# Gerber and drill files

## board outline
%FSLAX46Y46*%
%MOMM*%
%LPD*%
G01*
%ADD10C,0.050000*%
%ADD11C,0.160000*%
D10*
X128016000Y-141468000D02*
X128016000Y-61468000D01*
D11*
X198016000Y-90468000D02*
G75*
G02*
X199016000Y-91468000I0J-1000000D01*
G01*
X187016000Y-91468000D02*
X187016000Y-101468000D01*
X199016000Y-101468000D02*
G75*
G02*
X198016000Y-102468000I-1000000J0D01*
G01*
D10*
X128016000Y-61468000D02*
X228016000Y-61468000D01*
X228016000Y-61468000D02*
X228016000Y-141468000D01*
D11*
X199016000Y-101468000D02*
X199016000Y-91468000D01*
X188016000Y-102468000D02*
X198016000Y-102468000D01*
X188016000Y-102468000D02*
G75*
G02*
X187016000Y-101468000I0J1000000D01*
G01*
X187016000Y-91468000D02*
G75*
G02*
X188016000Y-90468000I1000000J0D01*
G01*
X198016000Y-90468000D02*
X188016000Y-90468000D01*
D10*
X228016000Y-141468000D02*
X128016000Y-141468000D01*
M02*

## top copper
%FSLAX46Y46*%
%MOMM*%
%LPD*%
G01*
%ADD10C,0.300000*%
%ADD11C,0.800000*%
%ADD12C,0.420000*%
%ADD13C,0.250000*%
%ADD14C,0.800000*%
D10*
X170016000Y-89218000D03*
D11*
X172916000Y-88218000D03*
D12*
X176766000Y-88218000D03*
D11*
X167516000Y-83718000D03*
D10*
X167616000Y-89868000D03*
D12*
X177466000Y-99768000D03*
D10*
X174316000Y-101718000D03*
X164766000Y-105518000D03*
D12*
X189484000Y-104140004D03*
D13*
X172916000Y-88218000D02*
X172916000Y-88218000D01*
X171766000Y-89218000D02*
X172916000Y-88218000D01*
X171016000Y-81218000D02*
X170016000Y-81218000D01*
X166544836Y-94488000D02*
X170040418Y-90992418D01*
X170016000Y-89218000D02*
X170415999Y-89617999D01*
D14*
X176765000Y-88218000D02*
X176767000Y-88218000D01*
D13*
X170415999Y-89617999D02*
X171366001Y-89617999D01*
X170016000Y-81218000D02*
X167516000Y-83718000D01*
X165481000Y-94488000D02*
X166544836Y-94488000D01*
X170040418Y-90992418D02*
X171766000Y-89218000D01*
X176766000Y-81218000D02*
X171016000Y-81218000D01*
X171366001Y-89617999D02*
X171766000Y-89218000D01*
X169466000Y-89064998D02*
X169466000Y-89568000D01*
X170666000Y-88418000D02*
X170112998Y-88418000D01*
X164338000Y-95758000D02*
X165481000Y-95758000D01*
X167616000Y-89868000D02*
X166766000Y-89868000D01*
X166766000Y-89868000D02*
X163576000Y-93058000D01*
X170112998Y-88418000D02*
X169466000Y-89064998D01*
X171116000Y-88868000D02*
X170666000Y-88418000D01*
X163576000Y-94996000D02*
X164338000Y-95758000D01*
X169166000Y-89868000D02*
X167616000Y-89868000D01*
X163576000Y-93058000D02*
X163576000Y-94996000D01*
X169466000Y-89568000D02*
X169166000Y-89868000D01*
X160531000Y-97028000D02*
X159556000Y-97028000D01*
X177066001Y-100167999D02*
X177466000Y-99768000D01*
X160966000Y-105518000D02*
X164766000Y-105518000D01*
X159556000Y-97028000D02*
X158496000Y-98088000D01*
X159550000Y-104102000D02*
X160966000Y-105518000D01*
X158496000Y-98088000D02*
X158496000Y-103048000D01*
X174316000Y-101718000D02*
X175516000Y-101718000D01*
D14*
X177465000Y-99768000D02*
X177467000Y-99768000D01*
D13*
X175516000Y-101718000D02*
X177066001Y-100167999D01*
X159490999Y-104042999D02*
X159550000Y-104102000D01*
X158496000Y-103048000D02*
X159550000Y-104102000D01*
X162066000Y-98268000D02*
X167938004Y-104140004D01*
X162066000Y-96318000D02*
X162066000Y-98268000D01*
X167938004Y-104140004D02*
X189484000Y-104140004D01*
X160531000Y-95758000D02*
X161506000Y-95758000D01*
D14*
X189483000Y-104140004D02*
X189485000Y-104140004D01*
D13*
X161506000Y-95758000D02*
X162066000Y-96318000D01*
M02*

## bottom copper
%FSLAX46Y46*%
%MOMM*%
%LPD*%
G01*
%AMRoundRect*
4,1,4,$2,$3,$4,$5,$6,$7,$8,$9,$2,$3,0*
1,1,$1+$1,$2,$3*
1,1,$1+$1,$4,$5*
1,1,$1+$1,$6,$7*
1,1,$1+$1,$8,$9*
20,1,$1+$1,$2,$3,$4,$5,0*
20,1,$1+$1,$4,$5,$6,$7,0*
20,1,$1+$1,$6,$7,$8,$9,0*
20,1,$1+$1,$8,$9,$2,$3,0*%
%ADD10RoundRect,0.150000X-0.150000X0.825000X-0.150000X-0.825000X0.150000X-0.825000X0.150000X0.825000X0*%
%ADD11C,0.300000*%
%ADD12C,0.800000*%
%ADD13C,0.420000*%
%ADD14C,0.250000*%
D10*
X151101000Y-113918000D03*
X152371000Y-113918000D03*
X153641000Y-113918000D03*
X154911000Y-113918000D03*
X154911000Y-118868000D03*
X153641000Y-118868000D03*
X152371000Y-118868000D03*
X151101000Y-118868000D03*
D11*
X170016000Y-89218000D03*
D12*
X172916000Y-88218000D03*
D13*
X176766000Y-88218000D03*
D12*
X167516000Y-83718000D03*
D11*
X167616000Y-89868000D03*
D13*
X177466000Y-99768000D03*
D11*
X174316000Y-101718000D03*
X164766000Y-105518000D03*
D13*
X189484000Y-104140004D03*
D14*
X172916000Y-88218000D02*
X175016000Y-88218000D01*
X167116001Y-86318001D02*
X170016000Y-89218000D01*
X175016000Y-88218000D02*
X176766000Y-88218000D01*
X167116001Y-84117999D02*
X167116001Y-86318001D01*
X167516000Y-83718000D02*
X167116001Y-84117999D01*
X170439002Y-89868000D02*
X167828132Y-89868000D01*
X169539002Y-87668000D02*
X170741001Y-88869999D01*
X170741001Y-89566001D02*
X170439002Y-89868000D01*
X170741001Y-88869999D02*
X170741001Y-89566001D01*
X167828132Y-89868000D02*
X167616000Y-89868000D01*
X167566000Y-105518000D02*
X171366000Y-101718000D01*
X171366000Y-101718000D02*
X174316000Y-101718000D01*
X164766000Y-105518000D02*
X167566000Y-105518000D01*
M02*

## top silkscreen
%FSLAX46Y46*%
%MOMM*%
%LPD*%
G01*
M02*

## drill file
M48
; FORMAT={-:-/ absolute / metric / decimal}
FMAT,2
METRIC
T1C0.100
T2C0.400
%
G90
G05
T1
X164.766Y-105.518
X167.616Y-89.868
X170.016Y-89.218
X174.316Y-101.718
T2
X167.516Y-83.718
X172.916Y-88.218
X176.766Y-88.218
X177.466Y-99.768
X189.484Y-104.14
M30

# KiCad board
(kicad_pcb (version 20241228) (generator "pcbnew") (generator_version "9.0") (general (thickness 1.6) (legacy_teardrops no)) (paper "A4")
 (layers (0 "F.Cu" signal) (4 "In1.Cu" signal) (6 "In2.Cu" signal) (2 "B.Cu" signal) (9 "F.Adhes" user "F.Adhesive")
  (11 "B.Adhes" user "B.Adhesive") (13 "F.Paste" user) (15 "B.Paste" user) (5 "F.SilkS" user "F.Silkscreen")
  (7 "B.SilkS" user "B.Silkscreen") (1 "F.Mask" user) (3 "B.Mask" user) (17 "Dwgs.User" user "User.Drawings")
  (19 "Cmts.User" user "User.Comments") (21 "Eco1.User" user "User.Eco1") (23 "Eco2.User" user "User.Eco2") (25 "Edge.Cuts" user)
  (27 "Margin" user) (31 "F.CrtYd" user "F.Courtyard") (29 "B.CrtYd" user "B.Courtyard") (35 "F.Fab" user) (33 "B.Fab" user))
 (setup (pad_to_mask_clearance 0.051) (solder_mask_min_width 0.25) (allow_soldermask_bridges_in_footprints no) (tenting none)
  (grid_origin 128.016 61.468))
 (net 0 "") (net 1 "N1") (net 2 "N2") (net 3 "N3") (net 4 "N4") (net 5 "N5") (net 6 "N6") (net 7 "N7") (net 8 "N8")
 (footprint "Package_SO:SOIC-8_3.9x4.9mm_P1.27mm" (layer "B.Cu") (at 153.006 116.393 -90)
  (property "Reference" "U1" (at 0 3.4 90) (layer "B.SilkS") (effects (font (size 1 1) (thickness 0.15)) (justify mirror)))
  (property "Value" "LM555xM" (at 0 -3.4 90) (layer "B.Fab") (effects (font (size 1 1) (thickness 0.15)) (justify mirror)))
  (pad "1" smd roundrect (at -2.475 1.905 270) (size 1.95 0.6) (layers "B.Cu" "B.Mask" "B.Paste") (roundrect_rratio 0.25) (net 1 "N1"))
  (pad "2" smd roundrect (at -2.475 0.635 270) (size 1.95 0.6) (layers "B.Cu" "B.Mask" "B.Paste") (roundrect_rratio 0.25) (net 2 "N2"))
  (pad "3" smd roundrect (at -2.475 -0.635 270) (size 1.95 0.6) (layers "B.Cu" "B.Mask" "B.Paste") (roundrect_rratio 0.25) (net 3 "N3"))
  (pad "4" smd roundrect (at -2.475 -1.905 270) (size 1.95 0.6) (layers "B.Cu" "B.Mask" "B.Paste") (roundrect_rratio 0.25) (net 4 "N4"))
  (pad "5" smd roundrect (at 2.475 -1.905 270) (size 1.95 0.6) (layers "B.Cu" "B.Mask" "B.Paste") (roundrect_rratio 0.25) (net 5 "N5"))
  (pad "6" smd roundrect (at 2.475 -0.635 270) (size 1.95 0.6) (layers "B.Cu" "B.Mask" "B.Paste") (roundrect_rratio 0.25) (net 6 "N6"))
  (pad "7" smd roundrect (at 2.475 0.635 270) (size 1.95 0.6) (layers "B.Cu" "B.Mask" "B.Paste") (roundrect_rratio 0.25) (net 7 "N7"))
  (pad "8" smd roundrect (at 2.475 1.905 270) (size 1.95 0.6) (layers "B.Cu" "B.Mask" "B.Paste") (roundrect_rratio 0.25) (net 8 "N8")))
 (gr_line (start 128.016 141.468) (end 128.016 61.468) (stroke (width 0.05) (type solid)) (layer "Edge.Cuts"))
 (gr_arc (start 198.016 90.468) (mid 198.723107 90.760893) (end 199.016 91.468) (stroke (width 0.16) (type solid)) (layer "Edge.Cuts"))
 (gr_line (start 187.016 91.468) (end 187.016 101.468) (stroke (width 0.16) (type solid)) (layer "Edge.Cuts"))
 (gr_arc (start 199.016 101.468) (mid 198.723107 102.175107) (end 198.016 102.468) (stroke (width 0.16) (type solid)) (layer "Edge.Cuts"))
 (gr_line (start 128.016 61.468) (end 228.016 61.468) (stroke (width 0.05) (type solid)) (layer "Edge.Cuts"))
 (gr_line (start 228.016 61.468) (end 228.016 141.468) (stroke (width 0.05) (type solid)) (layer "Edge.Cuts"))
 (gr_line (start 199.016 101.468) (end 199.016 91.468) (stroke (width 0.16) (type solid)) (layer "Edge.Cuts"))
 (gr_line (start 188.016 102.468) (end 198.016 102.468) (stroke (width 0.16) (type solid)) (layer "Edge.Cuts"))
 (gr_arc (start 188.016 102.468) (mid 187.308893 102.175107) (end 187.016 101.468) (stroke (width 0.16) (type solid)) (layer "Edge.Cuts"))
 (gr_arc (start 187.016 91.468) (mid 187.308893 90.760893) (end 188.016 90.468) (stroke (width 0.16) (type solid)) (layer "Edge.Cuts"))
 (gr_line (start 198.016 90.468) (end 188.016 90.468) (stroke (width 0.16) (type solid)) (layer "Edge.Cuts"))
 (gr_line (start 228.016 141.468) (end 128.016 141.468) (stroke (width 0.05) (type solid)) (layer "Edge.Cuts"))
 (segment (start 172.916 88.218) (end 172.916 88.218) (width 0.25) (layer "F.Cu") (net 8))
 (segment (start 171.766 89.218) (end 172.916 88.218) (width 0.25) (layer "F.Cu") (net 8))
 (segment (start 171.016 81.218) (end 170.016 81.218) (width 0.25) (layer "F.Cu") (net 8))
 (segment (start 166.544836 94.488) (end 170.040418 90.992418) (width 0.25) (layer "F.Cu") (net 8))
 (segment (start 170.016 89.218) (end 170.415999 89.617999) (width 0.25) (layer "F.Cu") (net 8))
 (segment (start 176.765 88.218) (end 176.767 88.218) (width 0.8) (layer "F.Cu") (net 8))
 (segment (start 170.415999 89.617999) (end 171.366001 89.617999) (width 0.25) (layer "F.Cu") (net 8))
 (segment (start 170.016 81.218) (end 167.516 83.718) (width 0.25) (layer "F.Cu") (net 8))
 (segment (start 165.481 94.488) (end 166.544836 94.488) (width 0.25) (layer "F.Cu") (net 8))
 (segment (start 170.040418 90.992418) (end 171.766 89.218) (width 0.25) (layer "F.Cu") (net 8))
 (segment (start 176.766 81.218) (end 171.016 81.218) (width 0.25) (layer "F.Cu") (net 8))
 (segment (start 171.366001 89.617999) (end 171.766 89.218) (width 0.25) (layer "F.Cu") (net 8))
 (via (at 170.016 89.218) (size 0.3) (drill 0.1) (layers "F.Cu" "B.Cu") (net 8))
 (via (at 172.916 88.218) (size 0.8) (drill 0.4) (layers "F.Cu" "B.Cu") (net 8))
 (via (at 176.766 88.218) (size 0.42) (drill 0.4) (layers "F.Cu" "B.Cu") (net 8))
 (via (at 167.516 83.718) (size 0.8) (drill 0.4) (layers "F.Cu" "B.Cu") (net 8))
 (segment (start 172.916 88.218) (end 175.016 88.218) (width 0.25) (layer "B.Cu") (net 8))
 (segment (start 167.116001 86.318001) (end 170.016 89.218) (width 0.25) (layer "B.Cu") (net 8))
 (segment (start 175.016 88.218) (end 176.766 88.218) (width 0.25) (layer "B.Cu") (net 8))
 (segment (start 167.116001 84.117999) (end 167.116001 86.318001) (width 0.25) (layer "B.Cu") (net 8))
 (segment (start 167.516 83.718) (end 167.116001 84.117999) (width 0.25) (layer "B.Cu") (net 8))
 (segment (start 169.466 89.064998) (end 169.466 89.568) (width 0.25) (layer "F.Cu") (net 7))
 (segment (start 170.666 88.418) (end 170.112998 88.418) (width 0.25) (layer "F.Cu") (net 7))
 (segment (start 164.338 95.758) (end 165.481 95.758) (width 0.25) (layer "F.Cu") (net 7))
 (segment (start 167.616 89.868) (end 166.766 89.868) (width 0.25) (layer "F.Cu") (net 7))
 (segment (start 166.766 89.868) (end 163.576 93.058) (width 0.25) (layer "F.Cu") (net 7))
 (segment (start 170.112998 88.418) (end 169.466 89.064998) (width 0.25) (layer "F.Cu") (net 7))
 (segment (start 171.116 88.868) (end 170.666 88.418) (width 0.25) (layer "F.Cu") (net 7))
 (segment (start 163.576 94.996) (end 164.338 95.758) (width 0.25) (layer "F.Cu") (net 7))
 (segment (start 169.166 89.868) (end 167.616 89.868) (width 0.25) (layer "F.Cu") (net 7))
 (segment (start 163.576 93.058) (end 163.576 94.996) (width 0.25) (layer "F.Cu") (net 7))
 (segment (start 169.466 89.568) (end 169.166 89.868) (width 0.25) (layer "F.Cu") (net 7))
 (via (at 167.616 89.868) (size 0.3) (drill 0.1) (layers "F.Cu" "B.Cu") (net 7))
 (segment (start 170.439002 89.868) (end 167.828132 89.868) (width 0.25) (layer "B.Cu") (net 7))
 (segment (start 169.539002 87.668) (end 170.741001 88.869999) (width 0.25) (layer "B.Cu") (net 7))
 (segment (start 170.741001 89.566001) (end 170.439002 89.868) (width 0.25) (layer "B.Cu") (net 7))
 (segment (start 170.741001 88.869999) (end 170.741001 89.566001) (width 0.25) (layer "B.Cu") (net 7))
 (segment (start 167.828132 89.868) (end 167.616 89.868) (width 0.25) (layer "B.Cu") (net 7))
 (segment (start 160.531 97.028) (end 159.556 97.028) (width 0.25) (layer "F.Cu") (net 3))
 (segment (start 177.066001 100.167999) (end 177.466 99.768) (width 0.25) (layer "F.Cu") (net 3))
 (segment (start 160.966 105.518) (end 164.766 105.518) (width 0.25) (layer "F.Cu") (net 3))
 (segment (start 159.556 97.028) (end 158.496 98.088) (width 0.25) (layer "F.Cu") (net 3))
 (segment (start 159.55 104.102) (end 160.966 105.518) (width 0.25) (layer "F.Cu") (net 3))
 (segment (start 158.496 98.088) (end 158.496 103.048) (width 0.25) (layer "F.Cu") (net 3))
 (segment (start 174.316 101.718) (end 175.516 101.718) (width 0.25) (layer "F.Cu") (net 3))
 (segment (start 177.465 99.768) (end 177.467 99.768) (width 0.8) (layer "F.Cu") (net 3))
 (segment (start 175.516 101.718) (end 177.066001 100.167999) (width 0.25) (layer "F.Cu") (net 3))
 (segment (start 159.490999 104.042999) (end 159.55 104.102) (width 0.25) (layer "F.Cu") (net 3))
 (segment (start 158.496 103.048) (end 159.55 104.102) (width 0.25) (layer "F.Cu") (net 3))
 (via (at 177.466 99.768) (size 0.42) (drill 0.4) (layers "F.Cu" "B.Cu") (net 3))
 (via (at 174.316 101.718) (size 0.3) (drill 0.1) (layers "F.Cu" "B.Cu") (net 3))
 (via (at 164.766 105.518) (size 0.3) (drill 0.1) (layers "F.Cu" "B.Cu") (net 3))
 (segment (start 167.566 105.518) (end 171.366 101.718) (width 0.25) (layer "B.Cu") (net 3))
 (segment (start 171.366 101.718) (end 174.316 101.718) (width 0.25) (layer "B.Cu") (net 3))
 (segment (start 164.766 105.518) (end 167.566 105.518) (width 0.25) (layer "B.Cu") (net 3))
 (segment (start 162.066 98.268) (end 167.938004 104.140004) (width 0.25) (layer "F.Cu") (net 2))
 (segment (start 162.066 96.318) (end 162.066 98.268) (width 0.25) (layer "F.Cu") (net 2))
 (segment (start 167.938004 104.140004) (end 189.484 104.140004) (width 0.25) (layer "F.Cu") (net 2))
 (segment (start 160.531 95.758) (end 161.506 95.758) (width 0.25) (layer "F.Cu") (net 2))
 (segment (start 189.483 104.140004) (end 189.485 104.140004) (width 0.8) (layer "F.Cu") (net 2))
 (segment (start 161.506 95.758) (end 162.066 96.318) (width 0.25) (layer "F.Cu") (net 2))
 (via (at 189.484 104.140004) (size 0.42) (drill 0.4) (layers "F.Cu" "B.Cu") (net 2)))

